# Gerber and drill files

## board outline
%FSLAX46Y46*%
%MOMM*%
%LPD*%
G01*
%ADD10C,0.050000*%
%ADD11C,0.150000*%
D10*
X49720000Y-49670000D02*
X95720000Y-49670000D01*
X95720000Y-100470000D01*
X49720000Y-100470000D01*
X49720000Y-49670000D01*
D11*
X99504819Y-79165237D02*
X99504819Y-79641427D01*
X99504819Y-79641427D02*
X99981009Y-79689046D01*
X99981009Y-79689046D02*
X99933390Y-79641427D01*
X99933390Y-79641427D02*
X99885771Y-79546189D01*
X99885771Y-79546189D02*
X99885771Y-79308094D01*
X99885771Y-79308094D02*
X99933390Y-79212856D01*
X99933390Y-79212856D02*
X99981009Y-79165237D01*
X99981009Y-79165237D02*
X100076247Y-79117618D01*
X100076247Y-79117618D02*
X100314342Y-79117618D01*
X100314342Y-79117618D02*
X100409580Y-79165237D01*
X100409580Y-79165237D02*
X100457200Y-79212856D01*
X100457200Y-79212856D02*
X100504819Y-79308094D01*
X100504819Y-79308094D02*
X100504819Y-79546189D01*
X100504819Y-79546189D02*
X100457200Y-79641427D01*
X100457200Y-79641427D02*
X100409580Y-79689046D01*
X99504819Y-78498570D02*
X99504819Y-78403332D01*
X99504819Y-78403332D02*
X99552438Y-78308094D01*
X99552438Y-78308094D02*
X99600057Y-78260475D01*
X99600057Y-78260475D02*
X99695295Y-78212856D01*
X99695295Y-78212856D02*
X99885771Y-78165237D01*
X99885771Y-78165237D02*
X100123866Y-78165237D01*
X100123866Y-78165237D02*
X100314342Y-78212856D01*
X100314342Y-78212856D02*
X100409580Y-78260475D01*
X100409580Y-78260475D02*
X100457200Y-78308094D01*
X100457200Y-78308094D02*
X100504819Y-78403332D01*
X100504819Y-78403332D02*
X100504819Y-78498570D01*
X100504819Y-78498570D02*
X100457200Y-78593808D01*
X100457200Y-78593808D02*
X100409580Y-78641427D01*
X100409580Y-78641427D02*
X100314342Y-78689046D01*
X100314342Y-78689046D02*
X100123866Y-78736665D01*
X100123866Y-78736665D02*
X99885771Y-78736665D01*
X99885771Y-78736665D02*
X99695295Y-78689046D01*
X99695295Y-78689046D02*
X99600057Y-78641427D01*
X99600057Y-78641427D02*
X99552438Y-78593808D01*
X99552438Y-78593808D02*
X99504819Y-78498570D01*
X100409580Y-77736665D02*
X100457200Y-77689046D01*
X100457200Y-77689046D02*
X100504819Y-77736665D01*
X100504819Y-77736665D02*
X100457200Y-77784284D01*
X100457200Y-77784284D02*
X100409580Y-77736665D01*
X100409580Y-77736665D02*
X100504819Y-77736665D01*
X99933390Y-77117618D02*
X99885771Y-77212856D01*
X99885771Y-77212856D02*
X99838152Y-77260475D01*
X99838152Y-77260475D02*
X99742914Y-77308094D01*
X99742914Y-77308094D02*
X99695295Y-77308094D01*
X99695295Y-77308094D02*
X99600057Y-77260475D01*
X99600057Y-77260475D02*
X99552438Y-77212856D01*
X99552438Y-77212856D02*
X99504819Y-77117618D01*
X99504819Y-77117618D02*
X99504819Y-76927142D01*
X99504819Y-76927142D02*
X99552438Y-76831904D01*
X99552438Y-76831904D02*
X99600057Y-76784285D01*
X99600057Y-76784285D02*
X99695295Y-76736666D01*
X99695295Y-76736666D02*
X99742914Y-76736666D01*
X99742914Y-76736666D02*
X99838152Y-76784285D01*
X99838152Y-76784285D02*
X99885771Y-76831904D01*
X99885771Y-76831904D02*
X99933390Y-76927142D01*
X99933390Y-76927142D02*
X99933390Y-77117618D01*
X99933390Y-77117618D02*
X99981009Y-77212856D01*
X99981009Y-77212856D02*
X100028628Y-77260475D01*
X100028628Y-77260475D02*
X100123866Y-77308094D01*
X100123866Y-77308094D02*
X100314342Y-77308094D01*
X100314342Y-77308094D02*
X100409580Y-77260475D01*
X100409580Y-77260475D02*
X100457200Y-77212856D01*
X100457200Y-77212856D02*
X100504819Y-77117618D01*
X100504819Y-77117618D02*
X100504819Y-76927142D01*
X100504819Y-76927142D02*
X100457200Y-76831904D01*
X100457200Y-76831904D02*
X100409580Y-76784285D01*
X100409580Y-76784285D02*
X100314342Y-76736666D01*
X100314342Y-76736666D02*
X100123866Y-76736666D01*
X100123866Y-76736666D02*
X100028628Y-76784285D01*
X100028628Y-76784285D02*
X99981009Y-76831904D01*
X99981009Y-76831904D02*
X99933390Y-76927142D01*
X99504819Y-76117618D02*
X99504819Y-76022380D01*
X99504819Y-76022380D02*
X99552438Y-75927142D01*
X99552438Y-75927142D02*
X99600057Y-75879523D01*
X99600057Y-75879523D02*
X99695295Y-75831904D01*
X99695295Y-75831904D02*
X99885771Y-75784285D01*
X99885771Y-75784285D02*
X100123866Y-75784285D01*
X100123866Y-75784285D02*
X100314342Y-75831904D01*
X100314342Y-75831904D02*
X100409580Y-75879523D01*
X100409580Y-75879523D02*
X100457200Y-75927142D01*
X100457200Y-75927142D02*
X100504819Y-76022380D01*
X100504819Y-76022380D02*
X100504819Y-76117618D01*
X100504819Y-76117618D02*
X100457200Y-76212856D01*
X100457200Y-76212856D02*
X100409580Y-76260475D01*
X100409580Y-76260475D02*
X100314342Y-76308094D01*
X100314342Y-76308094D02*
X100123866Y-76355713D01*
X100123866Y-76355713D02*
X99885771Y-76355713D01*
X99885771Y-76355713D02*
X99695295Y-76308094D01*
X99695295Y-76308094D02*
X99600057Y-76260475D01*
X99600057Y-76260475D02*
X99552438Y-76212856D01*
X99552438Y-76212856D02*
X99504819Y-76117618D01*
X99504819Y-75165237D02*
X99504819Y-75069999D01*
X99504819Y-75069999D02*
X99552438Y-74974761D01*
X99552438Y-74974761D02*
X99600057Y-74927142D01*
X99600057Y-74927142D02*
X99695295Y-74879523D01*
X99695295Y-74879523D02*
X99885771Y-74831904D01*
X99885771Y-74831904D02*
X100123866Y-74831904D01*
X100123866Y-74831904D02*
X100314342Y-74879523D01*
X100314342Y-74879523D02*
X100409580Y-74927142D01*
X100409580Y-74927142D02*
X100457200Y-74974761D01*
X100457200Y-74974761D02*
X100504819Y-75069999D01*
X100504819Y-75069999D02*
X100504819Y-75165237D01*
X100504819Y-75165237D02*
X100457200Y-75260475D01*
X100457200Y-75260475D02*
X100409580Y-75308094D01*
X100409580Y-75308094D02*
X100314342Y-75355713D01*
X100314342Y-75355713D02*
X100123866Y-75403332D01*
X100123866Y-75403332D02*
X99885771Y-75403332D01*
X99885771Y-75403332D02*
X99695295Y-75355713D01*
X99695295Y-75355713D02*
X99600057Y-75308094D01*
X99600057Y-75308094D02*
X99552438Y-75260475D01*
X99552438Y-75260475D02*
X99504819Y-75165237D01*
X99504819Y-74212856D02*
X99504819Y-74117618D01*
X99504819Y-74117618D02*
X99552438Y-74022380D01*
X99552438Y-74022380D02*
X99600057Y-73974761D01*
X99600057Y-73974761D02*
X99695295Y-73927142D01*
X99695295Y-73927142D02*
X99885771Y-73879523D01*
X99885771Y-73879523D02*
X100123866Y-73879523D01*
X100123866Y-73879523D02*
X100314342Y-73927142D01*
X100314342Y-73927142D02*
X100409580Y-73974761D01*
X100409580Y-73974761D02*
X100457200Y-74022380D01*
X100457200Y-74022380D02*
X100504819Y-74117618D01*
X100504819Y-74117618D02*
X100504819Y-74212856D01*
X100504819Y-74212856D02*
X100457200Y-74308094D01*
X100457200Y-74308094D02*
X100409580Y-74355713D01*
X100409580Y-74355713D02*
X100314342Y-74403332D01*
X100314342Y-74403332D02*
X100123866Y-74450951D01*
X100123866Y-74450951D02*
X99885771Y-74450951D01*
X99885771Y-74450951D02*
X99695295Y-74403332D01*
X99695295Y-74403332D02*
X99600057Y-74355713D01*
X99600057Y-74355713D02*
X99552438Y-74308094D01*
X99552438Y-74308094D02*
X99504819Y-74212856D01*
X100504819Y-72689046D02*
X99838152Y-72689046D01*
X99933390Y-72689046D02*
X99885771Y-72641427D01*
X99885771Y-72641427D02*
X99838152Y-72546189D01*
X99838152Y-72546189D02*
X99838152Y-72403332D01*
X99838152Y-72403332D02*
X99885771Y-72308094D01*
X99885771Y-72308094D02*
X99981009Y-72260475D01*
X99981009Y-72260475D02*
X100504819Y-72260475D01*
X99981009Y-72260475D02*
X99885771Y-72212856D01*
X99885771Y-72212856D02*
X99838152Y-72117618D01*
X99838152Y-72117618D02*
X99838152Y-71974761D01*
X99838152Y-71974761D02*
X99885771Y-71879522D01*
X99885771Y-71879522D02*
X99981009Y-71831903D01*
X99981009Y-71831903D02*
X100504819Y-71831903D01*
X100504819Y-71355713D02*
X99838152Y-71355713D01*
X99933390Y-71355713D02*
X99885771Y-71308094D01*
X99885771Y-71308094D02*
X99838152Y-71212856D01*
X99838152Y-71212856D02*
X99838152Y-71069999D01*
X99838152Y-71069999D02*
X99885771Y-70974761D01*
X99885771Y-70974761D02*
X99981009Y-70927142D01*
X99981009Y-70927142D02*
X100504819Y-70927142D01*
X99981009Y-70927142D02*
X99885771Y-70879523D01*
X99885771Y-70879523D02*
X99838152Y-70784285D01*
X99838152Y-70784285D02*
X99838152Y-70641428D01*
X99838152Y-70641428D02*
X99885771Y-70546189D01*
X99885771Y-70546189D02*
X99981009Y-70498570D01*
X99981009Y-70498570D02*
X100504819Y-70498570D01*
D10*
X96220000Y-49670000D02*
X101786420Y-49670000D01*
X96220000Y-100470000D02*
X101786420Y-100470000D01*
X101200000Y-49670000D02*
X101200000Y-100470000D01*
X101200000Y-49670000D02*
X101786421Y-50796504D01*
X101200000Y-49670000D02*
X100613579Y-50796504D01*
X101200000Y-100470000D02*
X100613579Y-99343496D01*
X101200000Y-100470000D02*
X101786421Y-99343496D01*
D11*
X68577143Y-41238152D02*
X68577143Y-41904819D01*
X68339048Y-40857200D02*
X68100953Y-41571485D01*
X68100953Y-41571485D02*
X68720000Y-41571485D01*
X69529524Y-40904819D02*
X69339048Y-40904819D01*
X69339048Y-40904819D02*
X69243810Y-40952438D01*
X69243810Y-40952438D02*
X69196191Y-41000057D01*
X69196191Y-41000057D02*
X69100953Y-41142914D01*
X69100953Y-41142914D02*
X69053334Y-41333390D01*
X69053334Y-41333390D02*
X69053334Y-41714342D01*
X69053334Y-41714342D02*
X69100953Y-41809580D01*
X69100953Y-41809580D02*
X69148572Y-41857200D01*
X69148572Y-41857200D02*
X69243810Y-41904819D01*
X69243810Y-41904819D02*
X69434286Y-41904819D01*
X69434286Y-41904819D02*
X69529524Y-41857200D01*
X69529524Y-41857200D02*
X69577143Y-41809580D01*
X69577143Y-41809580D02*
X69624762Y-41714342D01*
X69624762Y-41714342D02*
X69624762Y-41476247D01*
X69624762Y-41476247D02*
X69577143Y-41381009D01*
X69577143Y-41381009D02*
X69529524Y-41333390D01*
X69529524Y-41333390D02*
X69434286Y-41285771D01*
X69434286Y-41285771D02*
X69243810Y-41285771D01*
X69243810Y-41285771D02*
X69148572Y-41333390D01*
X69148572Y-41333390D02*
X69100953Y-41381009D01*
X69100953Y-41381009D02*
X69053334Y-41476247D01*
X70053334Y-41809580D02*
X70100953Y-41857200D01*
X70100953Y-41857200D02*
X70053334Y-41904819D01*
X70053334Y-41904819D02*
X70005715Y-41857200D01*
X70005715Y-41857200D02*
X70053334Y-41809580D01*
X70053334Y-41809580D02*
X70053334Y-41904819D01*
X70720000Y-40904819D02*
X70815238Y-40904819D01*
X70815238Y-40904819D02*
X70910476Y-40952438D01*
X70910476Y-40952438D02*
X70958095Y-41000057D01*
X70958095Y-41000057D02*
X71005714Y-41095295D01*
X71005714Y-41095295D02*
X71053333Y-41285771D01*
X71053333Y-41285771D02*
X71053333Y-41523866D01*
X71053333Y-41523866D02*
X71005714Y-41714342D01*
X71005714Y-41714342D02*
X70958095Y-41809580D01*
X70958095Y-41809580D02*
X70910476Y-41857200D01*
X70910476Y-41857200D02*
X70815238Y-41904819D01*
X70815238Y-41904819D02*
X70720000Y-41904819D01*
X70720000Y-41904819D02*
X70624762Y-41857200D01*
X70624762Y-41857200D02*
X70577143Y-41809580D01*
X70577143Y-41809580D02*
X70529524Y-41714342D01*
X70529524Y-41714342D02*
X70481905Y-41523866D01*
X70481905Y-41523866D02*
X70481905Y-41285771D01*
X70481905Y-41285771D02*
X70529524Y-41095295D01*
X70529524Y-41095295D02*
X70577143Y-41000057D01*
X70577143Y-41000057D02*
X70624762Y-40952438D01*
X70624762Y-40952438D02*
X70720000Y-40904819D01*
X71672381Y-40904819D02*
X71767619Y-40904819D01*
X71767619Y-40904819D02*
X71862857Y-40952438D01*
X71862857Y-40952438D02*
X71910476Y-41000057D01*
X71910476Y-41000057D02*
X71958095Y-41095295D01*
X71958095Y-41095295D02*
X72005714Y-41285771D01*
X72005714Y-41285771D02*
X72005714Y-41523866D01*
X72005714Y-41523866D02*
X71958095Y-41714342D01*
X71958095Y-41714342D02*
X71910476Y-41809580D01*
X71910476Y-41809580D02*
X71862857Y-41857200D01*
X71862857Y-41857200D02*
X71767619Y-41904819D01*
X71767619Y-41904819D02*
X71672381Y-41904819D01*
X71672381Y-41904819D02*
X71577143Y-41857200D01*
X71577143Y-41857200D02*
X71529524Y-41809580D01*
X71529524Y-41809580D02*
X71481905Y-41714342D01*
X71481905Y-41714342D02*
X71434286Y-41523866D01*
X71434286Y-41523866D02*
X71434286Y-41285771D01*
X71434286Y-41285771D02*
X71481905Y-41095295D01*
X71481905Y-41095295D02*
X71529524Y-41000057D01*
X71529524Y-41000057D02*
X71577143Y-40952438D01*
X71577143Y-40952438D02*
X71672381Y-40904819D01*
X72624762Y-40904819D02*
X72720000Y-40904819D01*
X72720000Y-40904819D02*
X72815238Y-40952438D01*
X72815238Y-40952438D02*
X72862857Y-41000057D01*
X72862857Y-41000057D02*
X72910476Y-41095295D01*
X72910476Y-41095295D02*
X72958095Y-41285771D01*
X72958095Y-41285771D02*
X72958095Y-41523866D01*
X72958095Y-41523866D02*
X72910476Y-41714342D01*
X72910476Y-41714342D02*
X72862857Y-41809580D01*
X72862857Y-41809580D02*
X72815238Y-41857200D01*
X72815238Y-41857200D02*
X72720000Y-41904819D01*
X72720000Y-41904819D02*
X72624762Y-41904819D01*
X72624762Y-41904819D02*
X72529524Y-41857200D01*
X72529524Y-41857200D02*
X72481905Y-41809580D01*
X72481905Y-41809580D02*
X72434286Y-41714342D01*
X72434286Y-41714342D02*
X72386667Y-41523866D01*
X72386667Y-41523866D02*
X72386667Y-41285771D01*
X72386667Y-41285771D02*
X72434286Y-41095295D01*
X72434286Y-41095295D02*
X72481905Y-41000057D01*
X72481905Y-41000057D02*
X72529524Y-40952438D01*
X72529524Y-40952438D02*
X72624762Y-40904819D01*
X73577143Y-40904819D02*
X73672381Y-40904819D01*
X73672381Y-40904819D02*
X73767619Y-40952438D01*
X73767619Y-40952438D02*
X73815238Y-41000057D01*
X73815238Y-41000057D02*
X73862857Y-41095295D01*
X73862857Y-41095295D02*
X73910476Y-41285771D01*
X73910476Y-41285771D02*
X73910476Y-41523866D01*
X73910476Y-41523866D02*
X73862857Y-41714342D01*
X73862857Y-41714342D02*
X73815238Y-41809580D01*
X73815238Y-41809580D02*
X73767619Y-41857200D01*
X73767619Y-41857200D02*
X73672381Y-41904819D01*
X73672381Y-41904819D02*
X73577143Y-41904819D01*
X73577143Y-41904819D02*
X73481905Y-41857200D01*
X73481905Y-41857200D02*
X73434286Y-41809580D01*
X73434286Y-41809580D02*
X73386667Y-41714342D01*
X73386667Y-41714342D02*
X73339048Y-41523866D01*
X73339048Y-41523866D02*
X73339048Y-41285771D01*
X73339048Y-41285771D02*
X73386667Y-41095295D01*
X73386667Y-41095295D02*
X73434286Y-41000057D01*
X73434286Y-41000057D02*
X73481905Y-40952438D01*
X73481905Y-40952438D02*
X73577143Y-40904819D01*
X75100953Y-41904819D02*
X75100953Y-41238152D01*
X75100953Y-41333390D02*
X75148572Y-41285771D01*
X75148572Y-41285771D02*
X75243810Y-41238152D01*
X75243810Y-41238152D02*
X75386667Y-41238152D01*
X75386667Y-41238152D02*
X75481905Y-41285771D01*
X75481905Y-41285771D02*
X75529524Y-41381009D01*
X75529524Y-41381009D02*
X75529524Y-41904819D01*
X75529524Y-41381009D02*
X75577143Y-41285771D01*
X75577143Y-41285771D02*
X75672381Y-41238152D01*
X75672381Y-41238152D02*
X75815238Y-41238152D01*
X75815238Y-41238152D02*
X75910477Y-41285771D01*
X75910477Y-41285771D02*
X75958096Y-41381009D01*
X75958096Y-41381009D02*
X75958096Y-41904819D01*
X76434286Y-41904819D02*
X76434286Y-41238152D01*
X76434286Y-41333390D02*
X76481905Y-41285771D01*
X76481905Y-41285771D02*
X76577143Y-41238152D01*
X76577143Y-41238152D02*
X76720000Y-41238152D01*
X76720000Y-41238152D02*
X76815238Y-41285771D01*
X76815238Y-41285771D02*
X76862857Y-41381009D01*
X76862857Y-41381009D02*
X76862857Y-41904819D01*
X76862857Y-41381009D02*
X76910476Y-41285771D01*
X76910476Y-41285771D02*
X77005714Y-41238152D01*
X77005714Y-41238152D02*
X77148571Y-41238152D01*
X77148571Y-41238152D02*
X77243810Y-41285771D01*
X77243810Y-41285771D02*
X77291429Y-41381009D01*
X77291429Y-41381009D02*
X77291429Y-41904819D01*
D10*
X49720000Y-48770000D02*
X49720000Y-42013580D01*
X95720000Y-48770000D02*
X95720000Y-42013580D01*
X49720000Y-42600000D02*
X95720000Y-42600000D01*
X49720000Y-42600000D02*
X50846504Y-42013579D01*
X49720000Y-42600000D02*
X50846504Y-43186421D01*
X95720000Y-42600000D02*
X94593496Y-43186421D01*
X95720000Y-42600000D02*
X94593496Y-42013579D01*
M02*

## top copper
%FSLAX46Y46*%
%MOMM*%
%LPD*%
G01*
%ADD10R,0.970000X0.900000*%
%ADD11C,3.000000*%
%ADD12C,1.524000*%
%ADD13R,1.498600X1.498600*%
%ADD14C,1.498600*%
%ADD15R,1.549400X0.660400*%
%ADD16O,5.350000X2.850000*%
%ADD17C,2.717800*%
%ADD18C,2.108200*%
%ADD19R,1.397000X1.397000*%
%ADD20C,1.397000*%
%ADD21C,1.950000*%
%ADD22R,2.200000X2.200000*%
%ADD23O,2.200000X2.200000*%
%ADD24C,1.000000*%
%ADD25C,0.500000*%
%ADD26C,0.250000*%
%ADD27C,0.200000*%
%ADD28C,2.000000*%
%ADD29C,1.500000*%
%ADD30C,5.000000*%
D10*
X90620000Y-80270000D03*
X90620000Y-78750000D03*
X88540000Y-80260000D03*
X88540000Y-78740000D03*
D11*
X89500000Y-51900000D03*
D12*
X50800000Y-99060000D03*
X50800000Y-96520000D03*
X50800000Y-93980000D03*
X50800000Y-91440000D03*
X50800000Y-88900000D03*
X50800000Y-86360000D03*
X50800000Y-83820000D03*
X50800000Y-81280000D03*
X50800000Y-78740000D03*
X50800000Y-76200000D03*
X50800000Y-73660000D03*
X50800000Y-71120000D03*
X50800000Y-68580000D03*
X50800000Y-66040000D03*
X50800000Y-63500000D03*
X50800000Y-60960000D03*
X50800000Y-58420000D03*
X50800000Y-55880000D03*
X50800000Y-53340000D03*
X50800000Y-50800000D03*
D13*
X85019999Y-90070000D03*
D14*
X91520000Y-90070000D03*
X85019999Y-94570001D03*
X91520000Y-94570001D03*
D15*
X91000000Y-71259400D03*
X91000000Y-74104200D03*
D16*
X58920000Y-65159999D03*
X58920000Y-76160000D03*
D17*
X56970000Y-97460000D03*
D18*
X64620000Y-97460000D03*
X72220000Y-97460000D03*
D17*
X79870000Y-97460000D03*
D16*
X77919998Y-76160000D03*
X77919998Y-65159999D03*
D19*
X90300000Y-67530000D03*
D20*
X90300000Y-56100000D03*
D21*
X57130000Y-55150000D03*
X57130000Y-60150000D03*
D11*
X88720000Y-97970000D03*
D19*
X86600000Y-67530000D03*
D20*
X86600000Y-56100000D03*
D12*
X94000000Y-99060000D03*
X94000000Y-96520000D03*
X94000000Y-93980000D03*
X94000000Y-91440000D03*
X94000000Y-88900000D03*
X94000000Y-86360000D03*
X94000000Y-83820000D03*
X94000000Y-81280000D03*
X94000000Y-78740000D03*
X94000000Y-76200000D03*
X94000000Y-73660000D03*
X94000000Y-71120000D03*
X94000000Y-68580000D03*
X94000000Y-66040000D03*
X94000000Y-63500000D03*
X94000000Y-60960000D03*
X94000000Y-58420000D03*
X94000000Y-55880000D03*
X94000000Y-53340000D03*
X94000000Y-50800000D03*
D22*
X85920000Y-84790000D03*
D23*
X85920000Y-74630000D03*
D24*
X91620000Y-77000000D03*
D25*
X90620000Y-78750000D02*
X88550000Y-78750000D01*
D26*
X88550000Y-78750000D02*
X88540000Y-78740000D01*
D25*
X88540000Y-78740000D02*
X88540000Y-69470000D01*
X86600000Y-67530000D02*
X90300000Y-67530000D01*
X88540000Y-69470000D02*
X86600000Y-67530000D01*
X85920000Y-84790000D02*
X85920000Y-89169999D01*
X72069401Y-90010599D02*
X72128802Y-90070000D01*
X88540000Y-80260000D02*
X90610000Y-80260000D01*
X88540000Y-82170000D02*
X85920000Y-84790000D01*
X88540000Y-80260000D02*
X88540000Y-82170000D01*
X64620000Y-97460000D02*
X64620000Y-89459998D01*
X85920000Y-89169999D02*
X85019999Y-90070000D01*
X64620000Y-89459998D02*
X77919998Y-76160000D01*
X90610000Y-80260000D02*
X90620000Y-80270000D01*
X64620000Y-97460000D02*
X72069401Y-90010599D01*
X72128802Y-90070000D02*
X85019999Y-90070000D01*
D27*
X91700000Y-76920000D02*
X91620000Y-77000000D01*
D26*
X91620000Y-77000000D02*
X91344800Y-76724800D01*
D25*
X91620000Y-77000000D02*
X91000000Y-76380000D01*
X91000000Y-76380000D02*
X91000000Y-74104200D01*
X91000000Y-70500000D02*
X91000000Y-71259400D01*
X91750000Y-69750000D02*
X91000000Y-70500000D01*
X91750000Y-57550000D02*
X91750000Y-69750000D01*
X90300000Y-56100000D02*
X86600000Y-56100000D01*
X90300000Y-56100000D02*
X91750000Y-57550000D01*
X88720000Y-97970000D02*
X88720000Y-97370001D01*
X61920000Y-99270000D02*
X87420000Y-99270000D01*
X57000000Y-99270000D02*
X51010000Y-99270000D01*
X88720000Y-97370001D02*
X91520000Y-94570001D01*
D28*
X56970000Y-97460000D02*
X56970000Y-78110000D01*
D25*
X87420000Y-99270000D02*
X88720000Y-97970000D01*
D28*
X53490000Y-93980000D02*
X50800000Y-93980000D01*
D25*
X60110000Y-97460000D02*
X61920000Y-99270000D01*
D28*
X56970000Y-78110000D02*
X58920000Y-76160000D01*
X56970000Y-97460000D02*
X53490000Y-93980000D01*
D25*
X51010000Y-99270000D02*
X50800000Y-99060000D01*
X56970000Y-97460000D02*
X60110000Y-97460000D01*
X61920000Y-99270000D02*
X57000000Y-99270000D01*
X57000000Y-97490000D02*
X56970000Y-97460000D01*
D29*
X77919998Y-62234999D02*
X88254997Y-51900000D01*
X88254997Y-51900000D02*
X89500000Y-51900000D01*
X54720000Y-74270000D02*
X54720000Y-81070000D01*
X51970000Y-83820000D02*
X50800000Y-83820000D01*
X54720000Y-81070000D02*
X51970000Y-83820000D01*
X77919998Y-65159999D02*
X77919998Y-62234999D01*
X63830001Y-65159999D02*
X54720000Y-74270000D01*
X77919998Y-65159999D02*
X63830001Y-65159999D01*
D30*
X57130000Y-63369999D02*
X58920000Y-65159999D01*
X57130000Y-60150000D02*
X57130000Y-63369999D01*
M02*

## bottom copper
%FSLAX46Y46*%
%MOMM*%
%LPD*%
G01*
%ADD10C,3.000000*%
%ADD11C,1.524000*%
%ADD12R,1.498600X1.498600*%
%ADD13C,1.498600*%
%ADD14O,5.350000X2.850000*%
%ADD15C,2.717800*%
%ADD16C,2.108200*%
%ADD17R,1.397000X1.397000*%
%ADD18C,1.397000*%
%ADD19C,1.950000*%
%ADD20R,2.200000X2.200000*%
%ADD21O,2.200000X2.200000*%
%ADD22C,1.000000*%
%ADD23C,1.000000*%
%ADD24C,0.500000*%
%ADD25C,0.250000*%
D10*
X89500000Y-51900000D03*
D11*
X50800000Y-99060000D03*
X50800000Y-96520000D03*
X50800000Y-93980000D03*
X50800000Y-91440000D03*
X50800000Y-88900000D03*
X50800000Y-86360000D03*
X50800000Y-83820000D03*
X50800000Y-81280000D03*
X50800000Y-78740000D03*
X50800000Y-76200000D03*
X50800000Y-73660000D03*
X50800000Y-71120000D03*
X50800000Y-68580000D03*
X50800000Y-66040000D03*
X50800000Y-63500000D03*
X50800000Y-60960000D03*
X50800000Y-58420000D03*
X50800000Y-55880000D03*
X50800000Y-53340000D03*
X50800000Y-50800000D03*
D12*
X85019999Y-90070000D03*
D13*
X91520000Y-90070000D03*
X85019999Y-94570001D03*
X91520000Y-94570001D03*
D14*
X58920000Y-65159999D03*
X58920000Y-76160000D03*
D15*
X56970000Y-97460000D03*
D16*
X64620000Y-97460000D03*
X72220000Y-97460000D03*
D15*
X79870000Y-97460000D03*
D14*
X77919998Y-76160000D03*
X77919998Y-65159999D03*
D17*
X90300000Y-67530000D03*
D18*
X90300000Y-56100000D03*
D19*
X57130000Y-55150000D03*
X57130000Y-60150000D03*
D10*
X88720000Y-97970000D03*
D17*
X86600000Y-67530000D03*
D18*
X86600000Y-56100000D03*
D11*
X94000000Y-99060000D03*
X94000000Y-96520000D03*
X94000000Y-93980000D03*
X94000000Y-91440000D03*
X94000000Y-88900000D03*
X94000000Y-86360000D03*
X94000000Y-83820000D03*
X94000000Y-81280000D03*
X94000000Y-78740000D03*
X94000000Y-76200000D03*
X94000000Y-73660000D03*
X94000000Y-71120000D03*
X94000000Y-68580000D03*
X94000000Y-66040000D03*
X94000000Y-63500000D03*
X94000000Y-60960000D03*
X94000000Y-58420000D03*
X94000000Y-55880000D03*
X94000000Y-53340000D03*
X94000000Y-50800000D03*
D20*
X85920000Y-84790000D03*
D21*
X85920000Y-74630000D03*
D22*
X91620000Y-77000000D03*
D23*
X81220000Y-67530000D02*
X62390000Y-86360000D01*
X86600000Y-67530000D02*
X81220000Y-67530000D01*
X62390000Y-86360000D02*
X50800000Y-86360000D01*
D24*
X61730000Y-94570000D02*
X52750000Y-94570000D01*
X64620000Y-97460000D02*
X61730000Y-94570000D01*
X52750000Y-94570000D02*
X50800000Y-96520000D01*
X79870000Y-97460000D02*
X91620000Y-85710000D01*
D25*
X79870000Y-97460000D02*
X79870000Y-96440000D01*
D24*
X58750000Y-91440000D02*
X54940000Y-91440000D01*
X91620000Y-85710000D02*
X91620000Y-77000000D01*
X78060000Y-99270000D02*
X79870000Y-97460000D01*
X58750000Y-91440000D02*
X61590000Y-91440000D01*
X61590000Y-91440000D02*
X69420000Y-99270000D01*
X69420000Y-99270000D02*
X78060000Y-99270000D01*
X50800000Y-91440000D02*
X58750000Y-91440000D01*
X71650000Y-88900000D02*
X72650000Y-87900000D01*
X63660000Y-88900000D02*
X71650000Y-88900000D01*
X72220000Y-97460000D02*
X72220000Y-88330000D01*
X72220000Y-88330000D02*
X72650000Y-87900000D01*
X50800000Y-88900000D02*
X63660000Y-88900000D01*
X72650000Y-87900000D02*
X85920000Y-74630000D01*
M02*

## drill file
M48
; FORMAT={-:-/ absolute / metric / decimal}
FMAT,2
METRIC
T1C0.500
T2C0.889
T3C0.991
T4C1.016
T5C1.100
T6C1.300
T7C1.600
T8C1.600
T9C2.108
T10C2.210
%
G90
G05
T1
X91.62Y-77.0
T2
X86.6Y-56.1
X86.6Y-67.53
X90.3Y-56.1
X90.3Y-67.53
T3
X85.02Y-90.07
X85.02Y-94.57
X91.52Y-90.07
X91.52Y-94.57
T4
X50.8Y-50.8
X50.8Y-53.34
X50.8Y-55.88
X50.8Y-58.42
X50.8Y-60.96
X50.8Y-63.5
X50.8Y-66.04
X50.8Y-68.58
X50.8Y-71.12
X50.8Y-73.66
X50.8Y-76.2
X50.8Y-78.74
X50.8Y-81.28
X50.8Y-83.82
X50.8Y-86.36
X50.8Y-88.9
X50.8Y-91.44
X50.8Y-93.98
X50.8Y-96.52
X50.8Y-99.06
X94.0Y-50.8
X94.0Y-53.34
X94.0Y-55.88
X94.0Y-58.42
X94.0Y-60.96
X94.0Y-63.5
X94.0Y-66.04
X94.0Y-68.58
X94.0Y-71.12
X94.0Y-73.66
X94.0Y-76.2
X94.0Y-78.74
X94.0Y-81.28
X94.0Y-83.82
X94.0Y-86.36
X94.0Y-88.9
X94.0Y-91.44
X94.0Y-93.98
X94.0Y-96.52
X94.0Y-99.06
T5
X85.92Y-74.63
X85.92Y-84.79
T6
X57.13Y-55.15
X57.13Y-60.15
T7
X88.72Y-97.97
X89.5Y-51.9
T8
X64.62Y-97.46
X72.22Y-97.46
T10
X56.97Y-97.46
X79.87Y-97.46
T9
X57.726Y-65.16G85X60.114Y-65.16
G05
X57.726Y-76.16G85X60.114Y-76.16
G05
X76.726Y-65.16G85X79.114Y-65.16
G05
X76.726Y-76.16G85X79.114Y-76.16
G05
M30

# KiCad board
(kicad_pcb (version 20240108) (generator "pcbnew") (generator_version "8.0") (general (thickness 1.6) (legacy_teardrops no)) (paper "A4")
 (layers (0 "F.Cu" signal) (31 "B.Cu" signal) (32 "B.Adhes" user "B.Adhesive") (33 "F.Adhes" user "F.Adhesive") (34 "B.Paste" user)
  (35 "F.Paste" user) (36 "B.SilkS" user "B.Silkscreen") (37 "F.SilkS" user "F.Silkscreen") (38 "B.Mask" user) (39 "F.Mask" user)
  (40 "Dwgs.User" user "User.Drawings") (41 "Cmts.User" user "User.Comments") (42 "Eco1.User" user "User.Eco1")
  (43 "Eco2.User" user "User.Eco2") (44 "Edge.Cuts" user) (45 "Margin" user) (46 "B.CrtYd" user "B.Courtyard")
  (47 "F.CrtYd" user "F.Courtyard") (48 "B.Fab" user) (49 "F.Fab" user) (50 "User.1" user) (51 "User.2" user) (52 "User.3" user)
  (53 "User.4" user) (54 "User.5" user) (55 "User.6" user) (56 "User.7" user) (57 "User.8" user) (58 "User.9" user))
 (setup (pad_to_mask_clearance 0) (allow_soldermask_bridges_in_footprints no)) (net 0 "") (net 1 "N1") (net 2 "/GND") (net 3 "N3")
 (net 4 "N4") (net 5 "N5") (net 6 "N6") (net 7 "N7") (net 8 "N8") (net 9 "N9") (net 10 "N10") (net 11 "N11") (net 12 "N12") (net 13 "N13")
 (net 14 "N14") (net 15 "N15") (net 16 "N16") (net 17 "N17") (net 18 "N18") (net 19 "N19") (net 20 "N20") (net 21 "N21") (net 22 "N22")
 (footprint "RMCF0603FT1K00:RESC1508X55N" (layer "F.Cu") (at 90.62 79.51 90)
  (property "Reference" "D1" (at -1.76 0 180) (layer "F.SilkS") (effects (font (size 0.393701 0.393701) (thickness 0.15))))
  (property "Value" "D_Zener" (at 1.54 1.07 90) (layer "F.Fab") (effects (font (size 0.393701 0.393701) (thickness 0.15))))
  (pad "1" smd rect (at -0.76 0 90) (size 0.9 0.97) (layers "F.Cu" "F.Paste" "F.Mask") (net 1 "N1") (solder_mask_margin 0.102))
  (pad "2" smd rect (at 0.76 0 90) (size 0.9 0.97) (layers "F.Cu" "F.Paste" "F.Mask") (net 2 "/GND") (solder_mask_margin 0.102)))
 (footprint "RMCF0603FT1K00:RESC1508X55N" (layer "F.Cu") (at 88.54 79.5 90)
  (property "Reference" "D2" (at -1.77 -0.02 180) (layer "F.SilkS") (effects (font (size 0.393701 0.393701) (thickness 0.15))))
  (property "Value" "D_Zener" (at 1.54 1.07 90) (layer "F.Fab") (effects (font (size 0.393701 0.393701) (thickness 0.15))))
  (pad "1" smd rect (at -0.76 0 90) (size 0.9 0.97) (layers "F.Cu" "F.Paste" "F.Mask") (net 1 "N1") (solder_mask_margin 0.102))
  (pad "2" smd rect (at 0.76 0 90) (size 0.9 0.97) (layers "F.Cu" "F.Paste" "F.Mask") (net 2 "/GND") (solder_mask_margin 0.102)))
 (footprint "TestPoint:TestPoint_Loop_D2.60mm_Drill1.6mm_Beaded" (layer "F.Cu") (at 89.5 51.9)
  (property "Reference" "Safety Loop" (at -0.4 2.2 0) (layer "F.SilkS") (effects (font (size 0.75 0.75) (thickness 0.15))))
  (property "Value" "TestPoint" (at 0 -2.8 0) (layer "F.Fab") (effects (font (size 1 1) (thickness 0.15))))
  (pad "1" thru_hole circle (at 0 0) (size 3 3) (drill 1.6) (layers "*.Cu" "*.Mask") (remove_unused_layers no) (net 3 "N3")))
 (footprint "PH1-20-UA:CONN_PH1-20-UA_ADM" (layer "F.Cu") (at 50.8 99.06 90)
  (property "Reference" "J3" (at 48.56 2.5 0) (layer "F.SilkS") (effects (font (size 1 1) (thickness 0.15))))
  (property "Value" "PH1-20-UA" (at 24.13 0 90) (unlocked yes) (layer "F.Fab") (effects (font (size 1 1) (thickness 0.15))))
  (pad "1" thru_hole circle (at 0 0 90) (size 1.524 1.524) (drill 1.016) (layers "*.Cu" "*.Mask") (remove_unused_layers no) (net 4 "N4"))
  (pad "2" thru_hole circle (at 2.54 0 90) (size 1.524 1.524) (drill 1.016) (layers "*.Cu" "*.Mask") (remove_unused_layers no) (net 1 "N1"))
  (pad "3" thru_hole circle (at 5.08 0 90) (size 1.524 1.524) (drill 1.016) (layers "*.Cu" "*.Mask") (remove_unused_layers no) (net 4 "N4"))
  (pad "4" thru_hole circle (at 7.62 0 90) (size 1.524 1.524) (drill 1.016) (layers "*.Cu" "*.Mask") (remove_unused_layers no) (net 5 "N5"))
  (pad "5" thru_hole circle (at 10.16 0 90) (size 1.524 1.524) (drill 1.016) (layers "*.Cu" "*.Mask") (remove_unused_layers no) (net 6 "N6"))
  (pad "6" thru_hole circle (at 12.7 0 90) (size 1.524 1.524) (drill 1.016) (layers "*.Cu" "*.Mask") (remove_unused_layers no)
   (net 2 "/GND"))
  (pad "7" thru_hole circle (at 15.24 0 90) (size 1.524 1.524) (drill 1.016) (layers "*.Cu" "*.Mask") (remove_unused_layers no) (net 3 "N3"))
  (pad "8" thru_hole circle (at 17.78 0 90) (size 1.524 1.524) (drill 1.016) (layers "*.Cu" "*.Mask") (remove_unused_layers no) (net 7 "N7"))
  (pad "9" thru_hole circle (at 20.32 0 90) (size 1.524 1.524) (drill 1.016) (layers "*.Cu" "*.Mask") (remove_unused_layers no) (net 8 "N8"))
  (pad "10" thru_hole circle (at 22.86 0 90) (size 1.524 1.524) (drill 1.016) (layers "*.Cu" "*.Mask") (remove_unused_layers no)
   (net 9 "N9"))
  (pad "11" thru_hole circle (at 25.4 0 90) (size 1.524 1.524) (drill 1.016) (layers "*.Cu" "*.Mask") (remove_unused_layers no)
   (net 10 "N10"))
  (pad "12" thru_hole circle (at 27.94 0 90) (size 1.524 1.524) (drill 1.016) (layers "*.Cu" "*.Mask") (remove_unused_layers no)
   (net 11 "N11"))
  (pad "13" thru_hole circle (at 30.48 0 90) (size 1.524 1.524) (drill 1.016) (layers "*.Cu" "*.Mask") (remove_unused_layers no)
   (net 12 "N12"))
  (pad "14" thru_hole circle (at 33.02 0 90) (size 1.524 1.524) (drill 1.016) (layers "*.Cu" "*.Mask") (remove_unused_layers no)
   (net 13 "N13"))
  (pad "15" thru_hole circle (at 35.56 0 90) (size 1.524 1.524) (drill 1.016) (layers "*.Cu" "*.Mask") (remove_unused_layers no)
   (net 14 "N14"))
  (pad "16" thru_hole circle (at 38.1 0 90) (size 1.524 1.524) (drill 1.016) (layers "*.Cu" "*.Mask") (remove_unused_layers no)
   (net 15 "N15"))
  (pad "17" thru_hole circle (at 40.64 0 90) (size 1.524 1.524) (drill 1.016) (layers "*.Cu" "*.Mask") (remove_unused_layers no)
   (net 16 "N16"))
  (pad "18" thru_hole circle (at 43.18 0 90) (size 1.524 1.524) (drill 1.016) (layers "*.Cu" "*.Mask") (remove_unused_layers no)
   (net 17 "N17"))
  (pad "19" thru_hole circle (at 45.72 0 90) (size 1.524 1.524) (drill 1.016) (layers "*.Cu" "*.Mask") (remove_unused_layers no)
   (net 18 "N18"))
  (pad "20" thru_hole circle (at 48.26 0 90) (size 1.524 1.524) (drill 1.016) (layers "*.Cu" "*.Mask") (remove_unused_layers no)
   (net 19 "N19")))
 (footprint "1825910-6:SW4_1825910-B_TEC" (layer "F.Cu") (at 91.52 94.570001)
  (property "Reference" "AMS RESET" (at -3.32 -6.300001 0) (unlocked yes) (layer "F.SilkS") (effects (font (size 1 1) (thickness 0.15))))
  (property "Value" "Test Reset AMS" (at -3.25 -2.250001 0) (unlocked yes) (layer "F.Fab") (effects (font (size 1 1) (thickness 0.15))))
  (pad "1" thru_hole rect (at -6.500001 -4.500001) (size 1.4986 1.4986) (drill 0.9906) (layers "*.Cu" "*.Mask") (remove_unused_layers no)
   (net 1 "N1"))
  (pad "2" thru_hole circle (at 0 -4.500001) (size 1.4986 1.4986) (drill 0.9906) (layers "*.Cu" "*.Mask") (remove_unused_layers no))
  (pad "3" thru_hole circle (at -6.500001 0) (size 1.4986 1.4986) (drill 0.9906) (layers "*.Cu" "*.Mask") (remove_unused_layers no))
  (pad "4" thru_hole circle (at 0 0) (size 1.4986 1.4986) (drill 0.9906) (layers "*.Cu" "*.Mask") (remove_unused_layers no) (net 4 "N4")))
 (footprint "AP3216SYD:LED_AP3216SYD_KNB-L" (layer "F.Cu") (at 91 72.6818 -90)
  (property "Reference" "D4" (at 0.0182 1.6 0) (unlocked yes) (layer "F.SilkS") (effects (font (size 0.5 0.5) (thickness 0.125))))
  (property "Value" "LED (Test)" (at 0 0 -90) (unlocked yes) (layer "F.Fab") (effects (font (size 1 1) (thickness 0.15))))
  (pad "1" smd rect (at -1.4224 0 270) (size 0.6604 1.5494) (layers "F.Cu" "F.Paste" "F.Mask") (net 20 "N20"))
  (pad "2" smd rect (at 1.4224 0 270) (size 0.6604 1.5494) (layers "F.Cu" "F.Paste" "F.Mask") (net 5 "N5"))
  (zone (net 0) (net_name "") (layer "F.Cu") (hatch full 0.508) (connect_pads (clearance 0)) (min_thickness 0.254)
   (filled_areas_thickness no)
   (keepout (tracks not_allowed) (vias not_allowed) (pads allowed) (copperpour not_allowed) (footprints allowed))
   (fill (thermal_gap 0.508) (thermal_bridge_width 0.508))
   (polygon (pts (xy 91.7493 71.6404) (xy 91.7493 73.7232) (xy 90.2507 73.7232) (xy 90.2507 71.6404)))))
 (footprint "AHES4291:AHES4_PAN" (layer "F.Cu") (at 58.919999 65.159998)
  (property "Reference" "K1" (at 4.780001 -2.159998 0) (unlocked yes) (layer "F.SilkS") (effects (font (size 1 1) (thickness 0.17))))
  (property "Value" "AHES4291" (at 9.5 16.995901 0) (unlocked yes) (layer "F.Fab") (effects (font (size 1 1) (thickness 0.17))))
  (pad "1" thru_hole oval (at 0.000001 0.000001) (size 5.35 2.85) (drill oval 4.4958 2.1082) (layers "*.Cu" "*.Mask")
   (remove_unused_layers no) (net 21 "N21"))
  (pad "2" thru_hole oval (at 0.000001 11.000002) (size 5.35 2.85) (drill oval 4.4958 2.1082) (layers "*.Cu" "*.Mask")
   (remove_unused_layers no) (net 4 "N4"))
  (pad "3" thru_hole circle (at -1.949999 32.300002) (size 2.7178 2.7178) (drill 2.2098) (layers "*.Cu" "*.Mask") (remove_unused_layers no)
   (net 4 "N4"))
  (pad "4" thru_hole circle (at 5.700001 32.300002) (size 2.1082 2.1082) (drill 1.6002) (layers "*.Cu" "*.Mask") (remove_unused_layers no)
   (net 1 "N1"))
  (pad "5" thru_hole circle (at 13.300001 32.300002) (size 2.1082 2.1082) (drill 1.6002) (layers "*.Cu" "*.Mask") (remove_unused_layers no)
   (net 6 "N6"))
  (pad "6" thru_hole circle (at 20.950001 32.300002) (size 2.7178 2.7178) (drill 2.2098) (layers "*.Cu" "*.Mask") (remove_unused_layers no)
   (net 5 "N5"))
  (pad "7" thru_hole oval (at 18.999999 11.000002) (size 5.35 2.85) (drill oval 4.4958 2.1082) (layers "*.Cu" "*.Mask")
   (remove_unused_layers no) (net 1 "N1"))
  (pad "8" thru_hole oval (at 18.999999 0.000001) (size 5.35 2.85) (drill oval 4.4958 2.1082) (layers "*.Cu" "*.Mask")
   (remove_unused_layers no) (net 3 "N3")))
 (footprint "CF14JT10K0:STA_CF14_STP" (layer "F.Cu") (at 90.3 67.53 90)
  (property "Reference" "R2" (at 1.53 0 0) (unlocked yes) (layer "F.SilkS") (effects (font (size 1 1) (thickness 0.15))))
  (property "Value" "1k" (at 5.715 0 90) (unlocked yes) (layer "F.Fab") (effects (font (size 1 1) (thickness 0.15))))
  (pad "1" thru_hole rect (at 0 0 90) (size 1.397 1.397) (drill 0.889) (layers "*.Cu" "*.Mask") (remove_unused_layers no) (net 2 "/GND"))
  (pad "2" thru_hole circle (at 11.43 0 90) (size 1.397 1.397) (drill 0.889) (layers "*.Cu" "*.Mask") (remove_unused_layers no)
   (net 20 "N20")))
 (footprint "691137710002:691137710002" (layer "F.Cu") (at 57.13 57.65 -90)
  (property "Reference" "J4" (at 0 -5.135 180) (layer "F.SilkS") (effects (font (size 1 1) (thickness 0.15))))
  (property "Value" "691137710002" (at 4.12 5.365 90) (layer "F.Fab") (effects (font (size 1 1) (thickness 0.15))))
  (pad "1" thru_hole circle (at -2.5 0 270) (size 1.95 1.95) (drill 1.3) (layers "*.Cu" "*.Mask") (remove_unused_layers no) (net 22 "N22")
   (solder_mask_margin 0.102))
  (pad "2" thru_hole circle (at 2.5 0 270) (size 1.95 1.95) (drill 1.3) (layers "*.Cu" "*.Mask") (remove_unused_layers no) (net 21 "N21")
   (solder_mask_margin 0.102)))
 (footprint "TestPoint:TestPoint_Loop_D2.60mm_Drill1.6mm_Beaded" (layer "F.Cu") (at 88.72 97.97)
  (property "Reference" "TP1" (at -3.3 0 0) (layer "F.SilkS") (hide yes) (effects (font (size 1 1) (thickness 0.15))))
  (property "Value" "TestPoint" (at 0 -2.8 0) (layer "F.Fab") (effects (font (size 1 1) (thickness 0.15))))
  (pad "1" thru_hole circle (at 0 0) (size 3 3) (drill 1.6) (layers "*.Cu" "*.Mask") (remove_unused_layers no) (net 4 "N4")))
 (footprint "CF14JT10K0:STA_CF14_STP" (layer "F.Cu") (at 86.6 67.53 90)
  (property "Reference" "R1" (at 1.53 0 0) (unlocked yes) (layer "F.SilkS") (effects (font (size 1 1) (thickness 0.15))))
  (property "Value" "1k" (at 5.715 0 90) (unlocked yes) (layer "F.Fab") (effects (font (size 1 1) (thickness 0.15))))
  (pad "1" thru_hole rect (at 0 0 90) (size 1.397 1.397) (drill 0.889) (layers "*.Cu" "*.Mask") (remove_unused_layers no) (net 2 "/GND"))
  (pad "2" thru_hole circle (at 11.43 0 90) (size 1.397 1.397) (drill 0.889) (layers "*.Cu" "*.Mask") (remove_unused_layers no)
   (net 20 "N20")))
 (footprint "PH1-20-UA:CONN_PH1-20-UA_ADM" (layer "F.Cu") (at 94 99.06 90)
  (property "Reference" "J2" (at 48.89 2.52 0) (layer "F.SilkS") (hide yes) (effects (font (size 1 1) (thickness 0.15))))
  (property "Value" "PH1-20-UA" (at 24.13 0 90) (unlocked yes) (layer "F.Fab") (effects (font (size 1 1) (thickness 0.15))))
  (pad "1" thru_hole circle (at 0 0 90) (size 1.524 1.524) (drill 1.016) (layers "*.Cu" "*.Mask") (remove_unused_layers no))
  (pad "2" thru_hole circle (at 2.54 0 90) (size 1.524 1.524) (drill 1.016) (layers "*.Cu" "*.Mask") (remove_unused_layers no))
  (pad "3" thru_hole circle (at 5.08 0 90) (size 1.524 1.524) (drill 1.016) (layers "*.Cu" "*.Mask") (remove_unused_layers no))
  (pad "4" thru_hole circle (at 7.62 0 90) (size 1.524 1.524) (drill 1.016) (layers "*.Cu" "*.Mask") (remove_unused_layers no))
  (pad "5" thru_hole circle (at 10.16 0 90) (size 1.524 1.524) (drill 1.016) (layers "*.Cu" "*.Mask") (remove_unused_layers no))
  (pad "6" thru_hole circle (at 12.7 0 90) (size 1.524 1.524) (drill 1.016) (layers "*.Cu" "*.Mask") (remove_unused_layers no))
  (pad "7" thru_hole circle (at 15.24 0 90) (size 1.524 1.524) (drill 1.016) (layers "*.Cu" "*.Mask") (remove_unused_layers no))
  (pad "8" thru_hole circle (at 17.78 0 90) (size 1.524 1.524) (drill 1.016) (layers "*.Cu" "*.Mask") (remove_unused_layers no))
  (pad "9" thru_hole circle (at 20.32 0 90) (size 1.524 1.524) (drill 1.016) (layers "*.Cu" "*.Mask") (remove_unused_layers no))
  (pad "10" thru_hole circle (at 22.86 0 90) (size 1.524 1.524) (drill 1.016) (layers "*.Cu" "*.Mask") (remove_unused_layers no))
  (pad "11" thru_hole circle (at 25.4 0 90) (size 1.524 1.524) (drill 1.016) (layers "*.Cu" "*.Mask") (remove_unused_layers no))
  (pad "12" thru_hole circle (at 27.94 0 90) (size 1.524 1.524) (drill 1.016) (layers "*.Cu" "*.Mask") (remove_unused_layers no))
  (pad "13" thru_hole circle (at 30.48 0 90) (size 1.524 1.524) (drill 1.016) (layers "*.Cu" "*.Mask") (remove_unused_layers no))
  (pad "14" thru_hole circle (at 33.02 0 90) (size 1.524 1.524) (drill 1.016) (layers "*.Cu" "*.Mask") (remove_unused_layers no))
  (pad "15" thru_hole circle (at 35.56 0 90) (size 1.524 1.524) (drill 1.016) (layers "*.Cu" "*.Mask") (remove_unused_layers no))
  (pad "16" thru_hole circle (at 38.1 0 90) (size 1.524 1.524) (drill 1.016) (layers "*.Cu" "*.Mask") (remove_unused_layers no))
  (pad "17" thru_hole circle (at 40.64 0 90) (size 1.524 1.524) (drill 1.016) (layers "*.Cu" "*.Mask") (remove_unused_layers no))
  (pad "18" thru_hole circle (at 43.18 0 90) (size 1.524 1.524) (drill 1.016) (layers "*.Cu" "*.Mask") (remove_unused_layers no))
  (pad "19" thru_hole circle (at 45.72 0 90) (size 1.524 1.524) (drill 1.016) (layers "*.Cu" "*.Mask") (remove_unused_layers no))
  (pad "20" thru_hole circle (at 48.26 0 90) (size 1.524 1.524) (drill 1.016) (layers "*.Cu" "*.Mask") (remove_unused_layers no)))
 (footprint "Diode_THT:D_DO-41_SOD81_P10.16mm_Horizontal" (layer "F.Cu") (at 85.92 84.79 90)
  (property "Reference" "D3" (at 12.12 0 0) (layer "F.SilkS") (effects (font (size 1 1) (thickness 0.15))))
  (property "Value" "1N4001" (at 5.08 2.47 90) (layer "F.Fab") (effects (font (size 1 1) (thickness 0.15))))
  (pad "1" thru_hole rect (at 0 0 90) (size 2.2 2.2) (drill 1.1) (layers "*.Cu" "*.Mask") (remove_unused_layers no) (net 1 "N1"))
  (pad "2" thru_hole oval (at 10.16 0 90) (size 2.2 2.2) (drill 1.1) (layers "*.Cu" "*.Mask") (remove_unused_layers no) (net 6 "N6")))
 (gr_rect (start 49.72 49.67) (end 95.72 100.47) (stroke (width 0.05) (type default)) (fill none) (layer "Edge.Cuts"))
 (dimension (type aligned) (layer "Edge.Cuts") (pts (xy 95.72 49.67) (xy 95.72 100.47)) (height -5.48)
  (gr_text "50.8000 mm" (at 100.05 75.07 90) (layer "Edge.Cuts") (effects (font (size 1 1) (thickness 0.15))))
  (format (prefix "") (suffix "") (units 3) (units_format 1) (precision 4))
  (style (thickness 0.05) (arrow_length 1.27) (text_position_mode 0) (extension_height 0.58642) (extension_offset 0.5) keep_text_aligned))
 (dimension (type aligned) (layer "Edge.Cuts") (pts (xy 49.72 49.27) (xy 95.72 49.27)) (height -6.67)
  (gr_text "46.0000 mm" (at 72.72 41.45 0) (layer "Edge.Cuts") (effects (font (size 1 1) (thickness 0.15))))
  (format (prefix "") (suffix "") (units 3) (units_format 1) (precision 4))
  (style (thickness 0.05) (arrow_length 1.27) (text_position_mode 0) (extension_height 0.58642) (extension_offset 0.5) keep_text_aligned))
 (segment (start 90.62 78.75) (end 88.55 78.75) (width 0.5) (layer "F.Cu") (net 2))
 (segment (start 88.55 78.75) (end 88.54 78.74) (width 0.25) (layer "F.Cu") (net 2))
 (segment (start 88.54 78.74) (end 88.54 69.47) (width 0.5) (layer "F.Cu") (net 2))
 (segment (start 86.6 67.53) (end 90.3 67.53) (width 0.5) (layer "F.Cu") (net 2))
 (segment (start 88.54 69.47) (end 86.6 67.53) (width 0.5) (layer "F.Cu") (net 2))
 (segment (start 81.22 67.53) (end 62.39 86.36) (width 1) (layer "B.Cu") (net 2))
 (segment (start 86.6 67.53) (end 81.22 67.53) (width 1) (layer "B.Cu") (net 2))
 (segment (start 62.39 86.36) (end 50.8 86.36) (width 1) (layer "B.Cu") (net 2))
 (segment (start 85.92 84.79) (end 85.92 89.169999) (width 0.5) (layer "F.Cu") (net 1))
 (segment (start 72.069401 90.010599) (end 72.128802 90.07) (width 0.5) (layer "F.Cu") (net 1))
 (segment (start 88.54 80.26) (end 90.61 80.26) (width 0.5) (layer "F.Cu") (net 1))
 (segment (start 88.54 82.17) (end 85.92 84.79) (width 0.5) (layer "F.Cu") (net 1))
 (segment (start 88.54 80.26) (end 88.54 82.17) (width 0.5) (layer "F.Cu") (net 1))
 (segment (start 64.62 97.46) (end 64.62 89.459998) (width 0.5) (layer "F.Cu") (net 1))
 (segment (start 85.92 89.169999) (end 85.019999 90.07) (width 0.5) (layer "F.Cu") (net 1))
 (segment (start 64.62 89.459998) (end 77.919998 76.16) (width 0.5) (layer "F.Cu") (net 1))
 (segment (start 90.61 80.26) (end 90.62 80.27) (width 0.5) (layer "F.Cu") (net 1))
 (segment (start 64.62 97.46) (end 72.069401 90.010599) (width 0.5) (layer "F.Cu") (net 1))
 (segment (start 72.128802 90.07) (end 85.019999 90.07) (width 0.5) (layer "F.Cu") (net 1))
 (segment (start 61.73 94.57) (end 52.75 94.57) (width 0.5) (layer "B.Cu") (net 1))
 (segment (start 64.62 97.46) (end 61.73 94.57) (width 0.5) (layer "B.Cu") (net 1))
 (segment (start 52.75 94.57) (end 50.8 96.52) (width 0.5) (layer "B.Cu") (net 1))
 (segment (start 91.7 76.92) (end 91.62 77) (width 0.2) (layer "F.Cu") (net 5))
 (segment (start 91.62 77) (end 91.3448 76.7248) (width 0.25) (layer "F.Cu") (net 5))
 (segment (start 91.62 77) (end 91 76.38) (width 0.5) (layer "F.Cu") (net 5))
 (segment (start 91 76.38) (end 91 74.1042) (width 0.5) (layer "F.Cu") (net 5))
 (via (at 91.62 77) (size 1) (drill 0.5) (layers "F.Cu" "B.Cu") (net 5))
 (segment (start 79.87 97.46) (end 91.62 85.71) (width 0.5) (layer "B.Cu") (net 5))
 (segment (start 79.87 97.46) (end 79.87 96.44) (width 0.25) (layer "B.Cu") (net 5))
 (segment (start 58.75 91.44) (end 54.94 91.44) (width 0.5) (layer "B.Cu") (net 5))
 (segment (start 91.62 85.71) (end 91.62 77) (width 0.5) (layer "B.Cu") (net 5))
 (segment (start 78.06 99.27) (end 79.87 97.46) (width 0.5) (layer "B.Cu") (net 5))
 (segment (start 58.75 91.44) (end 61.59 91.44) (width 0.5) (layer "B.Cu") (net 5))
 (segment (start 61.59 91.44) (end 69.42 99.27) (width 0.5) (layer "B.Cu") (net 5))
 (segment (start 69.42 99.27) (end 78.06 99.27) (width 0.5) (layer "B.Cu") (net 5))
 (segment (start 50.8 91.44) (end 58.75 91.44) (width 0.5) (layer "B.Cu") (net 5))
 (segment (start 71.65 88.9) (end 72.65 87.9) (width 0.5) (layer "B.Cu") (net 6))
 (segment (start 63.66 88.9) (end 71.65 88.9) (width 0.5) (layer "B.Cu") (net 6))
 (segment (start 72.22 97.46) (end 72.22 88.33) (width 0.5) (layer "B.Cu") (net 6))
 (segment (start 72.22 88.33) (end 72.65 87.9) (width 0.5) (layer "B.Cu") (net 6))
 (segment (start 50.8 88.9) (end 63.66 88.9) (width 0.5) (layer "B.Cu") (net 6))
 (segment (start 72.65 87.9) (end 85.92 74.63) (width 0.5) (layer "B.Cu") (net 6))
 (segment (start 91 70.5) (end 91 71.2594) (width 0.5) (layer "F.Cu") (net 20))
 (segment (start 91.75 69.75) (end 91 70.5) (width 0.5) (layer "F.Cu") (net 20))
 (segment (start 91.75 57.55) (end 91.75 69.75) (width 0.5) (layer "F.Cu") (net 20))
 (segment (start 90.3 56.1) (end 86.6 56.1) (width 0.5) (layer "F.Cu") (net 20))
 (segment (start 90.3 56.1) (end 91.75 57.55) (width 0.5) (layer "F.Cu") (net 20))
 (segment (start 88.72 97.97) (end 88.72 97.370001) (width 0.5) (layer "F.Cu") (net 4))
 (segment (start 61.92 99.27) (end 87.42 99.27) (width 0.5) (layer "F.Cu") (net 4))
 (segment (start 57 99.27) (end 51.01 99.27) (width 0.5) (layer "F.Cu") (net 4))
 (segment (start 88.72 97.370001) (end 91.52 94.570001) (width 0.5) (layer "F.Cu") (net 4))
 (segment (start 56.97 97.46) (end 56.97 78.11) (width 2) (layer "F.Cu") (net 4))
 (segment (start 87.42 99.27) (end 88.72 97.97) (width 0.5) (layer "F.Cu") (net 4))
 (segment (start 53.49 93.98) (end 50.8 93.98) (width 2) (layer "F.Cu") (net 4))
 (segment (start 60.11 97.46) (end 61.92 99.27) (width 0.5) (layer "F.Cu") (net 4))
 (segment (start 56.97 78.11) (end 58.92 76.16) (width 2) (layer "F.Cu") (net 4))
 (segment (start 56.97 97.46) (end 53.49 93.98) (width 2) (layer "F.Cu") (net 4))
 (segment (start 51.01 99.27) (end 50.8 99.06) (width 0.5) (layer "F.Cu") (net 4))
 (segment (start 56.97 97.46) (end 60.11 97.46) (width 0.5) (layer "F.Cu") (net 4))
 (segment (start 61.92 99.27) (end 57 99.27) (width 0.5) (layer "F.Cu") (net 4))
 (segment (start 57 97.49) (end 56.97 97.46) (width 0.5) (layer "F.Cu") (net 4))
 (segment (start 77.919998 62.234999) (end 88.254997 51.9) (width 1.5) (layer "F.Cu") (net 3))
 (segment (start 88.254997 51.9) (end 89.5 51.9) (width 1.5) (layer "F.Cu") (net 3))
 (segment (start 54.72 74.27) (end 54.72 81.07) (width 1.5) (layer "F.Cu") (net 3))
 (segment (start 51.97 83.82) (end 50.8 83.82) (width 1.5) (layer "F.Cu") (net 3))
 (segment (start 54.72 81.07) (end 51.97 83.82) (width 1.5) (layer "F.Cu") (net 3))
 (segment (start 77.919998 65.159999) (end 77.919998 62.234999) (width 1.5) (layer "F.Cu") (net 3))
 (segment (start 63.830001 65.159999) (end 54.72 74.27) (width 1.5) (layer "F.Cu") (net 3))
 (segment (start 77.919998 65.159999) (end 63.830001 65.159999) (width 1.5) (layer "F.Cu") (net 3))
 (segment (start 57.13 63.369999) (end 58.92 65.159999) (width 5) (layer "F.Cu") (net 21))
 (segment (start 57.13 60.15) (end 57.13 63.369999) (width 5) (layer "F.Cu") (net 21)))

